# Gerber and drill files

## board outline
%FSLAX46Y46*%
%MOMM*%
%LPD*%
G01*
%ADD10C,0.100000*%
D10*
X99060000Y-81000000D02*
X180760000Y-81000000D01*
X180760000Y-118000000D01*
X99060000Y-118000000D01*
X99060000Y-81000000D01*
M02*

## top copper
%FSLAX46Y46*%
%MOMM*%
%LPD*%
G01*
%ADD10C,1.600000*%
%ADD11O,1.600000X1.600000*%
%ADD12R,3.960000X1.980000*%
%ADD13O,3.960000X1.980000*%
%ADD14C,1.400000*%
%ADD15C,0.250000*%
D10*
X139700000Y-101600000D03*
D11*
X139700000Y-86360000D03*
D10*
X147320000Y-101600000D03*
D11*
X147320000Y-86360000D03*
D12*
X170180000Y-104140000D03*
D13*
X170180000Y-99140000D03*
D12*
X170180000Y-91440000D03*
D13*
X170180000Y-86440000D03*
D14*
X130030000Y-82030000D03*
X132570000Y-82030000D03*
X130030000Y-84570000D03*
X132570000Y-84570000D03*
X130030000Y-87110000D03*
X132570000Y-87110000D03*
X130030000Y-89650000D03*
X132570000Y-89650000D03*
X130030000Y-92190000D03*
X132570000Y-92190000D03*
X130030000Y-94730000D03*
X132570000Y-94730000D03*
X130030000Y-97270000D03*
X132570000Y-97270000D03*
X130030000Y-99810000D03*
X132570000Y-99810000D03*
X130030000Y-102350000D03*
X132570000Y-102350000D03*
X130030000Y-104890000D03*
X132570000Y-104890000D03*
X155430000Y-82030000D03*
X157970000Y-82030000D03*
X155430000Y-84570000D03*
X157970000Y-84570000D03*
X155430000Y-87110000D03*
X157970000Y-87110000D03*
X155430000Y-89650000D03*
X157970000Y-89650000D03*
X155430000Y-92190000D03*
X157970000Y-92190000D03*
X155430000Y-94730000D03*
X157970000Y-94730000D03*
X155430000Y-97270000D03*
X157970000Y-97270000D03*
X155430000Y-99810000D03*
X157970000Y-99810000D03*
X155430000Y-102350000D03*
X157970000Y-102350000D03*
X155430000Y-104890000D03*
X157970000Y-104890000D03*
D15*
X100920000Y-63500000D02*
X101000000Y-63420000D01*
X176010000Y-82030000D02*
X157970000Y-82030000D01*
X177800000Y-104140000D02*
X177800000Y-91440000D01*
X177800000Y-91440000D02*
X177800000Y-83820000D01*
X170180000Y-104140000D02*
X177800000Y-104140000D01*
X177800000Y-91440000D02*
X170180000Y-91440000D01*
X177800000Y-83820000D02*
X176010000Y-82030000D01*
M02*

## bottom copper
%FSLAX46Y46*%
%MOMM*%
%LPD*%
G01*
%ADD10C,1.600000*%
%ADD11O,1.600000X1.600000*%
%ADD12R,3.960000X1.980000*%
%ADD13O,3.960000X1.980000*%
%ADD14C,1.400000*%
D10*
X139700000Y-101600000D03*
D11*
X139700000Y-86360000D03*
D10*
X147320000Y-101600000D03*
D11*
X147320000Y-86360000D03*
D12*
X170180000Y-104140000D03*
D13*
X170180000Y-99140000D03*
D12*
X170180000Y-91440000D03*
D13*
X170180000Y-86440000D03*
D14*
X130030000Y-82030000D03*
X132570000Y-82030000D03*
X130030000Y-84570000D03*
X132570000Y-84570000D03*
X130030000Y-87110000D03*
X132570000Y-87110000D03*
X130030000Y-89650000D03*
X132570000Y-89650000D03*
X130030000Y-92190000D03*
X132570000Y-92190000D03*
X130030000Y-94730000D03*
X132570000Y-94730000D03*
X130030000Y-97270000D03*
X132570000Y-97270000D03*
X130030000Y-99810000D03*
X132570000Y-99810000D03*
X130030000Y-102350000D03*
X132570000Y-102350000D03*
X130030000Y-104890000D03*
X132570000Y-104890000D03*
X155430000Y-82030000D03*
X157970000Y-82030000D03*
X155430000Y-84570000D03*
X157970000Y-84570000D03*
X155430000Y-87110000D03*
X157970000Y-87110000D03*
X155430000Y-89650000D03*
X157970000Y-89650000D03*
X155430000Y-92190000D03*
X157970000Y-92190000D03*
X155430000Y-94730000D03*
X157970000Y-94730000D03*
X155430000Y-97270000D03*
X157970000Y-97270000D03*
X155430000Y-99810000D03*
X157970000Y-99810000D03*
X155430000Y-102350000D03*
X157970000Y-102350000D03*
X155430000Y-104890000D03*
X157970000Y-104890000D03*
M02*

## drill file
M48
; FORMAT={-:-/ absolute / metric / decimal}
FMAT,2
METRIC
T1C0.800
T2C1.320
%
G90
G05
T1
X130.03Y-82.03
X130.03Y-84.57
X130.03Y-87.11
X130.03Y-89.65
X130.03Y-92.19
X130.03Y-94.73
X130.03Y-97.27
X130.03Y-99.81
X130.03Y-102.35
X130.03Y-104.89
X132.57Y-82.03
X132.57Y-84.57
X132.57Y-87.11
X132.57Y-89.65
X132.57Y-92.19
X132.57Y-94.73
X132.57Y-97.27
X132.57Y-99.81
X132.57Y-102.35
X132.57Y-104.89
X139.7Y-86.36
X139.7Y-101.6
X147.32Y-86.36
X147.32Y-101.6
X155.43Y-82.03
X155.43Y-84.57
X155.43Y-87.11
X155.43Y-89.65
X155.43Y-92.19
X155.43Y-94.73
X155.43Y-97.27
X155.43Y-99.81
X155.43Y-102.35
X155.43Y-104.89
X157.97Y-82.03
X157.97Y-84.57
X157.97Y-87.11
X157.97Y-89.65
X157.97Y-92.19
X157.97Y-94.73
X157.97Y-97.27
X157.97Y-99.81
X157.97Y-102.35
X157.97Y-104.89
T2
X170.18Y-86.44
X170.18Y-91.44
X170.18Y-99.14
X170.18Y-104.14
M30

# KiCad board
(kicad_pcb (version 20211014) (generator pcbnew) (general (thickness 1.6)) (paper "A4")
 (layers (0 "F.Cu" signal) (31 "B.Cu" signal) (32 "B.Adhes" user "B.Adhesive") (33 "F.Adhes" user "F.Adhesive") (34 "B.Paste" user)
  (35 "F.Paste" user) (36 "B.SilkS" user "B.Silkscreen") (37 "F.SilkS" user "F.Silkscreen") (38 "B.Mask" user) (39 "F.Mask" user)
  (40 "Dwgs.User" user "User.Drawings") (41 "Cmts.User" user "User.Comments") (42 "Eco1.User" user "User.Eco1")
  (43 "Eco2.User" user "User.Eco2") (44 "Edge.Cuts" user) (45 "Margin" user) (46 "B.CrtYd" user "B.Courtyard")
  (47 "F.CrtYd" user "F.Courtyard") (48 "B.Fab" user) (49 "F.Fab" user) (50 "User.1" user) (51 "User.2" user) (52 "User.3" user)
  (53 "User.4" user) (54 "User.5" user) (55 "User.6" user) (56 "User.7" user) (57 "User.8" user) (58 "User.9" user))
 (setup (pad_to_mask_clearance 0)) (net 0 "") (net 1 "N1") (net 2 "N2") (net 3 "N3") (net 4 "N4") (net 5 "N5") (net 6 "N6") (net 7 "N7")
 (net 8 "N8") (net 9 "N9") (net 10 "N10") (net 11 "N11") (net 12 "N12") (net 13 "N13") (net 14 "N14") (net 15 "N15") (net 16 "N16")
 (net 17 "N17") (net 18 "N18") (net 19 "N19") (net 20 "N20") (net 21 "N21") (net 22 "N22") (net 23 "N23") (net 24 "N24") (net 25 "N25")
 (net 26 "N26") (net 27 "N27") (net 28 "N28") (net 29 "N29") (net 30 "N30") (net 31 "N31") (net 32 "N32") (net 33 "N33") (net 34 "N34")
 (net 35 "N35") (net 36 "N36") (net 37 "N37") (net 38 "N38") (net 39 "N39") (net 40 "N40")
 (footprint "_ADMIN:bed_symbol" (layer "F.Cu") (at 155 114)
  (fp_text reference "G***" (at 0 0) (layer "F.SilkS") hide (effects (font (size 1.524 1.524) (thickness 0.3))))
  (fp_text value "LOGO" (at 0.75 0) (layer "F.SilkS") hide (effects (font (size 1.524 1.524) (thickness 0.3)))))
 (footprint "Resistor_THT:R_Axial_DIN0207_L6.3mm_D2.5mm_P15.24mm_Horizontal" (layer "F.Cu") (at 139.7 101.6 90)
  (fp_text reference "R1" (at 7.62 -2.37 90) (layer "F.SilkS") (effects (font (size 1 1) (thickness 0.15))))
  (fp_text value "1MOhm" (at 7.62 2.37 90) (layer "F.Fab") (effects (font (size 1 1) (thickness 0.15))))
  (pad "1" thru_hole circle (at 0 0 90) (size 1.6 1.6) (drill 0.8) (layers *.Cu *.Mask) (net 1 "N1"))
  (pad "2" thru_hole oval (at 15.24 0 90) (size 1.6 1.6) (drill 0.8) (layers *.Cu *.Mask) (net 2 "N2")))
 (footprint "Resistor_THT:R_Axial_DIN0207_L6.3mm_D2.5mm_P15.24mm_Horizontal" (layer "F.Cu") (at 147.32 101.6 90)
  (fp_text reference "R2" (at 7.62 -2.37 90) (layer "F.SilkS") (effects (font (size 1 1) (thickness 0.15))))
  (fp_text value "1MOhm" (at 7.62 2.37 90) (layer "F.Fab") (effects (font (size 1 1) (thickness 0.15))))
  (pad "1" thru_hole circle (at 0 0 90) (size 1.6 1.6) (drill 0.8) (layers *.Cu *.Mask) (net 1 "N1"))
  (pad "2" thru_hole oval (at 15.24 0 90) (size 1.6 1.6) (drill 0.8) (layers *.Cu *.Mask) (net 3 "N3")))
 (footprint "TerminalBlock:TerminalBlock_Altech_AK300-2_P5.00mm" (layer "F.Cu") (at 170.18 104.14 90)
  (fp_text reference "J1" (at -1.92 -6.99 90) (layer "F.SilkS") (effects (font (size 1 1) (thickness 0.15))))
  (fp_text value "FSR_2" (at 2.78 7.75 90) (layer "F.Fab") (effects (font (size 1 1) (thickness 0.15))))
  (pad "1" thru_hole rect (at 0 0 90) (size 1.98 3.96) (drill 1.32) (layers *.Cu *.Mask) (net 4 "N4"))
  (pad "2" thru_hole oval (at 5 0 90) (size 1.98 3.96) (drill 1.32) (layers *.Cu *.Mask) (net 2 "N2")))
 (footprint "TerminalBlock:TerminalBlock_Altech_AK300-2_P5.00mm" (layer "F.Cu") (at 170.18 91.44 90)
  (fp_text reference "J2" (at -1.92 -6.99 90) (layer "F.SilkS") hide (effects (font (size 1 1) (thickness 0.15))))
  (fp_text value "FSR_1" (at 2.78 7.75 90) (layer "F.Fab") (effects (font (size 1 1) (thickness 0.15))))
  (pad "1" thru_hole rect (at 0 0 90) (size 1.98 3.96) (drill 1.32) (layers *.Cu *.Mask) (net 4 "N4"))
  (pad "2" thru_hole oval (at 5 0 90) (size 1.98 3.96) (drill 1.32) (layers *.Cu *.Mask) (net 3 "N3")))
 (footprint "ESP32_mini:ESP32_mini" (layer "F.Cu") (at 144 93.46)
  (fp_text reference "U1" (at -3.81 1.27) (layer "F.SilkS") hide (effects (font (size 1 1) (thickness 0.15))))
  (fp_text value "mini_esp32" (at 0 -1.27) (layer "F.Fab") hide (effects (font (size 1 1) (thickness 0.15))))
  (pad "1" thru_hole circle locked (at -13.97 -11.43 270) (size 1.4 1.4) (drill 0.8) (layers *.Cu *.Mask) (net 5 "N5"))
  (pad "2" thru_hole circle locked (at -11.43 -11.43 270) (size 1.4 1.4) (drill 0.8) (layers *.Cu *.Mask) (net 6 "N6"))
  (pad "3" thru_hole circle locked (at -13.97 -8.89 270) (size 1.4 1.4) (drill 0.8) (layers *.Cu *.Mask) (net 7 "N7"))
  (pad "4" thru_hole circle locked (at -11.43 -8.89 270) (size 1.4 1.4) (drill 0.8) (layers *.Cu *.Mask) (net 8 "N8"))
  (pad "5" thru_hole circle locked (at -13.97 -6.35 270) (size 1.4 1.4) (drill 0.8) (layers *.Cu *.Mask) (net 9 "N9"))
  (pad "6" thru_hole circle locked (at -11.43 -6.35 270) (size 1.4 1.4) (drill 0.8) (layers *.Cu *.Mask) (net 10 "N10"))
  (pad "7" thru_hole circle locked (at -13.97 -3.81 270) (size 1.4 1.4) (drill 0.8) (layers *.Cu *.Mask) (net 2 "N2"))
  (pad "8" thru_hole circle locked (at -11.43 -3.81 270) (size 1.4 1.4) (drill 0.8) (layers *.Cu *.Mask) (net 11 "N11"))
  (pad "9" thru_hole circle locked (at -13.97 -1.27 270) (size 1.4 1.4) (drill 0.8) (layers *.Cu *.Mask) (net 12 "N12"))
  (pad "10" thru_hole circle locked (at -11.43 -1.27 270) (size 1.4 1.4) (drill 0.8) (layers *.Cu *.Mask) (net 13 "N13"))
  (pad "11" thru_hole circle locked (at -13.97 1.27 270) (size 1.4 1.4) (drill 0.8) (layers *.Cu *.Mask) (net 3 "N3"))
  (pad "12" thru_hole circle locked (at -11.43 1.27 270) (size 1.4 1.4) (drill 0.8) (layers *.Cu *.Mask) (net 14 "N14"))
  (pad "13" thru_hole circle locked (at -13.97 3.81 270) (size 1.4 1.4) (drill 0.8) (layers *.Cu *.Mask) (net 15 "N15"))
  (pad "14" thru_hole circle locked (at -11.43 3.81 270) (size 1.4 1.4) (drill 0.8) (layers *.Cu *.Mask) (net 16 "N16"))
  (pad "15" thru_hole circle locked (at -13.97 6.35 270) (size 1.4 1.4) (drill 0.8) (layers *.Cu *.Mask) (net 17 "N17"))
  (pad "16" thru_hole circle locked (at -11.43 6.35 270) (size 1.4 1.4) (drill 0.8) (layers *.Cu *.Mask) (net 1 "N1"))
  (pad "17" thru_hole circle locked (at -13.97 8.89 270) (size 1.4 1.4) (drill 0.8) (layers *.Cu *.Mask) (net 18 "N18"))
  (pad "18" thru_hole circle locked (at -11.43 8.89 270) (size 1.4 1.4) (drill 0.8) (layers *.Cu *.Mask) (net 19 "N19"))
  (pad "19" thru_hole circle locked (at -13.97 11.43 270) (size 1.4 1.4) (drill 0.8) (layers *.Cu *.Mask) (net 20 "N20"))
  (pad "20" thru_hole circle locked (at -11.43 11.43 270) (size 1.4 1.4) (drill 0.8) (layers *.Cu *.Mask) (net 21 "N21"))
  (pad "21" thru_hole circle locked (at 11.43 -11.43 270) (size 1.4 1.4) (drill 0.8) (layers *.Cu *.Mask) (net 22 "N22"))
  (pad "22" thru_hole circle locked (at 13.97 -11.43 270) (size 1.4 1.4) (drill 0.8) (layers *.Cu *.Mask) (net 4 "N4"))
  (pad "23" thru_hole circle locked (at 11.43 -8.89 270) (size 1.4 1.4) (drill 0.8) (layers *.Cu *.Mask) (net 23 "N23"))
  (pad "24" thru_hole circle locked (at 13.97 -8.89 270) (size 1.4 1.4) (drill 0.8) (layers *.Cu *.Mask) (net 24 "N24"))
  (pad "25" thru_hole circle locked (at 11.43 -6.35 270) (size 1.4 1.4) (drill 0.8) (layers *.Cu *.Mask) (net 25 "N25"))
  (pad "26" thru_hole circle locked (at 13.97 -6.35 270) (size 1.4 1.4) (drill 0.8) (layers *.Cu *.Mask) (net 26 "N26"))
  (pad "27" thru_hole circle locked (at 11.43 -3.81 270) (size 1.4 1.4) (drill 0.8) (layers *.Cu *.Mask) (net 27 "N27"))
  (pad "28" thru_hole circle locked (at 13.97 -3.81 270) (size 1.4 1.4) (drill 0.8) (layers *.Cu *.Mask) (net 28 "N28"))
  (pad "29" thru_hole circle locked (at 11.43 -1.27 270) (size 1.4 1.4) (drill 0.8) (layers *.Cu *.Mask) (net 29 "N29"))
  (pad "30" thru_hole circle locked (at 13.97 -1.27 270) (size 1.4 1.4) (drill 0.8) (layers *.Cu *.Mask) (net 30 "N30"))
  (pad "31" thru_hole circle locked (at 11.43 1.27 270) (size 1.4 1.4) (drill 0.8) (layers *.Cu *.Mask) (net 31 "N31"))
  (pad "32" thru_hole circle locked (at 13.97 1.27 270) (size 1.4 1.4) (drill 0.8) (layers *.Cu *.Mask) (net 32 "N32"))
  (pad "33" thru_hole circle locked (at 11.43 3.81 270) (size 1.4 1.4) (drill 0.8) (layers *.Cu *.Mask) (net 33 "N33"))
  (pad "34" thru_hole circle locked (at 13.97 3.81 270) (size 1.4 1.4) (drill 0.8) (layers *.Cu *.Mask) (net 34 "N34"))
  (pad "35" thru_hole circle locked (at 11.43 6.35 270) (size 1.4 1.4) (drill 0.8) (layers *.Cu *.Mask) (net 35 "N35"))
  (pad "36" thru_hole circle locked (at 13.97 6.35 270) (size 1.4 1.4) (drill 0.8) (layers *.Cu *.Mask) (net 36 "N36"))
  (pad "37" thru_hole circle locked (at 11.43 8.89 270) (size 1.4 1.4) (drill 0.8) (layers *.Cu *.Mask) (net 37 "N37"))
  (pad "38" thru_hole circle locked (at 13.97 8.89 270) (size 1.4 1.4) (drill 0.8) (layers *.Cu *.Mask) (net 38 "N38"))
  (pad "39" thru_hole circle locked (at 11.43 11.43 270) (size 1.4 1.4) (drill 0.8) (layers *.Cu *.Mask) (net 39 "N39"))
  (pad "40" thru_hole circle locked (at 13.97 11.43 270) (size 1.4 1.4) (drill 0.8) (layers *.Cu *.Mask) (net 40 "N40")))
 (gr_rect (start 99.06 81) (end 180.76 118) (layer "Edge.Cuts") (width 0.1) (fill none))
 (segment (start 100.92 63.5) (end 101 63.42) (width 0.25) (layer "F.Cu") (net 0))
 (segment (start 176.01 82.03) (end 157.97 82.03) (width 0.25) (layer "F.Cu") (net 4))
 (segment (start 177.8 104.14) (end 177.8 91.44) (width 0.25) (layer "F.Cu") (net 4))
 (segment (start 177.8 91.44) (end 177.8 83.82) (width 0.25) (layer "F.Cu") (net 4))
 (segment (start 170.18 104.14) (end 177.8 104.14) (width 0.25) (layer "F.Cu") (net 4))
 (segment (start 177.8 91.44) (end 170.18 91.44) (width 0.25) (layer "F.Cu") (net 4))
 (segment (start 177.8 83.82) (end 176.01 82.03) (width 0.25) (layer "F.Cu") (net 4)))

